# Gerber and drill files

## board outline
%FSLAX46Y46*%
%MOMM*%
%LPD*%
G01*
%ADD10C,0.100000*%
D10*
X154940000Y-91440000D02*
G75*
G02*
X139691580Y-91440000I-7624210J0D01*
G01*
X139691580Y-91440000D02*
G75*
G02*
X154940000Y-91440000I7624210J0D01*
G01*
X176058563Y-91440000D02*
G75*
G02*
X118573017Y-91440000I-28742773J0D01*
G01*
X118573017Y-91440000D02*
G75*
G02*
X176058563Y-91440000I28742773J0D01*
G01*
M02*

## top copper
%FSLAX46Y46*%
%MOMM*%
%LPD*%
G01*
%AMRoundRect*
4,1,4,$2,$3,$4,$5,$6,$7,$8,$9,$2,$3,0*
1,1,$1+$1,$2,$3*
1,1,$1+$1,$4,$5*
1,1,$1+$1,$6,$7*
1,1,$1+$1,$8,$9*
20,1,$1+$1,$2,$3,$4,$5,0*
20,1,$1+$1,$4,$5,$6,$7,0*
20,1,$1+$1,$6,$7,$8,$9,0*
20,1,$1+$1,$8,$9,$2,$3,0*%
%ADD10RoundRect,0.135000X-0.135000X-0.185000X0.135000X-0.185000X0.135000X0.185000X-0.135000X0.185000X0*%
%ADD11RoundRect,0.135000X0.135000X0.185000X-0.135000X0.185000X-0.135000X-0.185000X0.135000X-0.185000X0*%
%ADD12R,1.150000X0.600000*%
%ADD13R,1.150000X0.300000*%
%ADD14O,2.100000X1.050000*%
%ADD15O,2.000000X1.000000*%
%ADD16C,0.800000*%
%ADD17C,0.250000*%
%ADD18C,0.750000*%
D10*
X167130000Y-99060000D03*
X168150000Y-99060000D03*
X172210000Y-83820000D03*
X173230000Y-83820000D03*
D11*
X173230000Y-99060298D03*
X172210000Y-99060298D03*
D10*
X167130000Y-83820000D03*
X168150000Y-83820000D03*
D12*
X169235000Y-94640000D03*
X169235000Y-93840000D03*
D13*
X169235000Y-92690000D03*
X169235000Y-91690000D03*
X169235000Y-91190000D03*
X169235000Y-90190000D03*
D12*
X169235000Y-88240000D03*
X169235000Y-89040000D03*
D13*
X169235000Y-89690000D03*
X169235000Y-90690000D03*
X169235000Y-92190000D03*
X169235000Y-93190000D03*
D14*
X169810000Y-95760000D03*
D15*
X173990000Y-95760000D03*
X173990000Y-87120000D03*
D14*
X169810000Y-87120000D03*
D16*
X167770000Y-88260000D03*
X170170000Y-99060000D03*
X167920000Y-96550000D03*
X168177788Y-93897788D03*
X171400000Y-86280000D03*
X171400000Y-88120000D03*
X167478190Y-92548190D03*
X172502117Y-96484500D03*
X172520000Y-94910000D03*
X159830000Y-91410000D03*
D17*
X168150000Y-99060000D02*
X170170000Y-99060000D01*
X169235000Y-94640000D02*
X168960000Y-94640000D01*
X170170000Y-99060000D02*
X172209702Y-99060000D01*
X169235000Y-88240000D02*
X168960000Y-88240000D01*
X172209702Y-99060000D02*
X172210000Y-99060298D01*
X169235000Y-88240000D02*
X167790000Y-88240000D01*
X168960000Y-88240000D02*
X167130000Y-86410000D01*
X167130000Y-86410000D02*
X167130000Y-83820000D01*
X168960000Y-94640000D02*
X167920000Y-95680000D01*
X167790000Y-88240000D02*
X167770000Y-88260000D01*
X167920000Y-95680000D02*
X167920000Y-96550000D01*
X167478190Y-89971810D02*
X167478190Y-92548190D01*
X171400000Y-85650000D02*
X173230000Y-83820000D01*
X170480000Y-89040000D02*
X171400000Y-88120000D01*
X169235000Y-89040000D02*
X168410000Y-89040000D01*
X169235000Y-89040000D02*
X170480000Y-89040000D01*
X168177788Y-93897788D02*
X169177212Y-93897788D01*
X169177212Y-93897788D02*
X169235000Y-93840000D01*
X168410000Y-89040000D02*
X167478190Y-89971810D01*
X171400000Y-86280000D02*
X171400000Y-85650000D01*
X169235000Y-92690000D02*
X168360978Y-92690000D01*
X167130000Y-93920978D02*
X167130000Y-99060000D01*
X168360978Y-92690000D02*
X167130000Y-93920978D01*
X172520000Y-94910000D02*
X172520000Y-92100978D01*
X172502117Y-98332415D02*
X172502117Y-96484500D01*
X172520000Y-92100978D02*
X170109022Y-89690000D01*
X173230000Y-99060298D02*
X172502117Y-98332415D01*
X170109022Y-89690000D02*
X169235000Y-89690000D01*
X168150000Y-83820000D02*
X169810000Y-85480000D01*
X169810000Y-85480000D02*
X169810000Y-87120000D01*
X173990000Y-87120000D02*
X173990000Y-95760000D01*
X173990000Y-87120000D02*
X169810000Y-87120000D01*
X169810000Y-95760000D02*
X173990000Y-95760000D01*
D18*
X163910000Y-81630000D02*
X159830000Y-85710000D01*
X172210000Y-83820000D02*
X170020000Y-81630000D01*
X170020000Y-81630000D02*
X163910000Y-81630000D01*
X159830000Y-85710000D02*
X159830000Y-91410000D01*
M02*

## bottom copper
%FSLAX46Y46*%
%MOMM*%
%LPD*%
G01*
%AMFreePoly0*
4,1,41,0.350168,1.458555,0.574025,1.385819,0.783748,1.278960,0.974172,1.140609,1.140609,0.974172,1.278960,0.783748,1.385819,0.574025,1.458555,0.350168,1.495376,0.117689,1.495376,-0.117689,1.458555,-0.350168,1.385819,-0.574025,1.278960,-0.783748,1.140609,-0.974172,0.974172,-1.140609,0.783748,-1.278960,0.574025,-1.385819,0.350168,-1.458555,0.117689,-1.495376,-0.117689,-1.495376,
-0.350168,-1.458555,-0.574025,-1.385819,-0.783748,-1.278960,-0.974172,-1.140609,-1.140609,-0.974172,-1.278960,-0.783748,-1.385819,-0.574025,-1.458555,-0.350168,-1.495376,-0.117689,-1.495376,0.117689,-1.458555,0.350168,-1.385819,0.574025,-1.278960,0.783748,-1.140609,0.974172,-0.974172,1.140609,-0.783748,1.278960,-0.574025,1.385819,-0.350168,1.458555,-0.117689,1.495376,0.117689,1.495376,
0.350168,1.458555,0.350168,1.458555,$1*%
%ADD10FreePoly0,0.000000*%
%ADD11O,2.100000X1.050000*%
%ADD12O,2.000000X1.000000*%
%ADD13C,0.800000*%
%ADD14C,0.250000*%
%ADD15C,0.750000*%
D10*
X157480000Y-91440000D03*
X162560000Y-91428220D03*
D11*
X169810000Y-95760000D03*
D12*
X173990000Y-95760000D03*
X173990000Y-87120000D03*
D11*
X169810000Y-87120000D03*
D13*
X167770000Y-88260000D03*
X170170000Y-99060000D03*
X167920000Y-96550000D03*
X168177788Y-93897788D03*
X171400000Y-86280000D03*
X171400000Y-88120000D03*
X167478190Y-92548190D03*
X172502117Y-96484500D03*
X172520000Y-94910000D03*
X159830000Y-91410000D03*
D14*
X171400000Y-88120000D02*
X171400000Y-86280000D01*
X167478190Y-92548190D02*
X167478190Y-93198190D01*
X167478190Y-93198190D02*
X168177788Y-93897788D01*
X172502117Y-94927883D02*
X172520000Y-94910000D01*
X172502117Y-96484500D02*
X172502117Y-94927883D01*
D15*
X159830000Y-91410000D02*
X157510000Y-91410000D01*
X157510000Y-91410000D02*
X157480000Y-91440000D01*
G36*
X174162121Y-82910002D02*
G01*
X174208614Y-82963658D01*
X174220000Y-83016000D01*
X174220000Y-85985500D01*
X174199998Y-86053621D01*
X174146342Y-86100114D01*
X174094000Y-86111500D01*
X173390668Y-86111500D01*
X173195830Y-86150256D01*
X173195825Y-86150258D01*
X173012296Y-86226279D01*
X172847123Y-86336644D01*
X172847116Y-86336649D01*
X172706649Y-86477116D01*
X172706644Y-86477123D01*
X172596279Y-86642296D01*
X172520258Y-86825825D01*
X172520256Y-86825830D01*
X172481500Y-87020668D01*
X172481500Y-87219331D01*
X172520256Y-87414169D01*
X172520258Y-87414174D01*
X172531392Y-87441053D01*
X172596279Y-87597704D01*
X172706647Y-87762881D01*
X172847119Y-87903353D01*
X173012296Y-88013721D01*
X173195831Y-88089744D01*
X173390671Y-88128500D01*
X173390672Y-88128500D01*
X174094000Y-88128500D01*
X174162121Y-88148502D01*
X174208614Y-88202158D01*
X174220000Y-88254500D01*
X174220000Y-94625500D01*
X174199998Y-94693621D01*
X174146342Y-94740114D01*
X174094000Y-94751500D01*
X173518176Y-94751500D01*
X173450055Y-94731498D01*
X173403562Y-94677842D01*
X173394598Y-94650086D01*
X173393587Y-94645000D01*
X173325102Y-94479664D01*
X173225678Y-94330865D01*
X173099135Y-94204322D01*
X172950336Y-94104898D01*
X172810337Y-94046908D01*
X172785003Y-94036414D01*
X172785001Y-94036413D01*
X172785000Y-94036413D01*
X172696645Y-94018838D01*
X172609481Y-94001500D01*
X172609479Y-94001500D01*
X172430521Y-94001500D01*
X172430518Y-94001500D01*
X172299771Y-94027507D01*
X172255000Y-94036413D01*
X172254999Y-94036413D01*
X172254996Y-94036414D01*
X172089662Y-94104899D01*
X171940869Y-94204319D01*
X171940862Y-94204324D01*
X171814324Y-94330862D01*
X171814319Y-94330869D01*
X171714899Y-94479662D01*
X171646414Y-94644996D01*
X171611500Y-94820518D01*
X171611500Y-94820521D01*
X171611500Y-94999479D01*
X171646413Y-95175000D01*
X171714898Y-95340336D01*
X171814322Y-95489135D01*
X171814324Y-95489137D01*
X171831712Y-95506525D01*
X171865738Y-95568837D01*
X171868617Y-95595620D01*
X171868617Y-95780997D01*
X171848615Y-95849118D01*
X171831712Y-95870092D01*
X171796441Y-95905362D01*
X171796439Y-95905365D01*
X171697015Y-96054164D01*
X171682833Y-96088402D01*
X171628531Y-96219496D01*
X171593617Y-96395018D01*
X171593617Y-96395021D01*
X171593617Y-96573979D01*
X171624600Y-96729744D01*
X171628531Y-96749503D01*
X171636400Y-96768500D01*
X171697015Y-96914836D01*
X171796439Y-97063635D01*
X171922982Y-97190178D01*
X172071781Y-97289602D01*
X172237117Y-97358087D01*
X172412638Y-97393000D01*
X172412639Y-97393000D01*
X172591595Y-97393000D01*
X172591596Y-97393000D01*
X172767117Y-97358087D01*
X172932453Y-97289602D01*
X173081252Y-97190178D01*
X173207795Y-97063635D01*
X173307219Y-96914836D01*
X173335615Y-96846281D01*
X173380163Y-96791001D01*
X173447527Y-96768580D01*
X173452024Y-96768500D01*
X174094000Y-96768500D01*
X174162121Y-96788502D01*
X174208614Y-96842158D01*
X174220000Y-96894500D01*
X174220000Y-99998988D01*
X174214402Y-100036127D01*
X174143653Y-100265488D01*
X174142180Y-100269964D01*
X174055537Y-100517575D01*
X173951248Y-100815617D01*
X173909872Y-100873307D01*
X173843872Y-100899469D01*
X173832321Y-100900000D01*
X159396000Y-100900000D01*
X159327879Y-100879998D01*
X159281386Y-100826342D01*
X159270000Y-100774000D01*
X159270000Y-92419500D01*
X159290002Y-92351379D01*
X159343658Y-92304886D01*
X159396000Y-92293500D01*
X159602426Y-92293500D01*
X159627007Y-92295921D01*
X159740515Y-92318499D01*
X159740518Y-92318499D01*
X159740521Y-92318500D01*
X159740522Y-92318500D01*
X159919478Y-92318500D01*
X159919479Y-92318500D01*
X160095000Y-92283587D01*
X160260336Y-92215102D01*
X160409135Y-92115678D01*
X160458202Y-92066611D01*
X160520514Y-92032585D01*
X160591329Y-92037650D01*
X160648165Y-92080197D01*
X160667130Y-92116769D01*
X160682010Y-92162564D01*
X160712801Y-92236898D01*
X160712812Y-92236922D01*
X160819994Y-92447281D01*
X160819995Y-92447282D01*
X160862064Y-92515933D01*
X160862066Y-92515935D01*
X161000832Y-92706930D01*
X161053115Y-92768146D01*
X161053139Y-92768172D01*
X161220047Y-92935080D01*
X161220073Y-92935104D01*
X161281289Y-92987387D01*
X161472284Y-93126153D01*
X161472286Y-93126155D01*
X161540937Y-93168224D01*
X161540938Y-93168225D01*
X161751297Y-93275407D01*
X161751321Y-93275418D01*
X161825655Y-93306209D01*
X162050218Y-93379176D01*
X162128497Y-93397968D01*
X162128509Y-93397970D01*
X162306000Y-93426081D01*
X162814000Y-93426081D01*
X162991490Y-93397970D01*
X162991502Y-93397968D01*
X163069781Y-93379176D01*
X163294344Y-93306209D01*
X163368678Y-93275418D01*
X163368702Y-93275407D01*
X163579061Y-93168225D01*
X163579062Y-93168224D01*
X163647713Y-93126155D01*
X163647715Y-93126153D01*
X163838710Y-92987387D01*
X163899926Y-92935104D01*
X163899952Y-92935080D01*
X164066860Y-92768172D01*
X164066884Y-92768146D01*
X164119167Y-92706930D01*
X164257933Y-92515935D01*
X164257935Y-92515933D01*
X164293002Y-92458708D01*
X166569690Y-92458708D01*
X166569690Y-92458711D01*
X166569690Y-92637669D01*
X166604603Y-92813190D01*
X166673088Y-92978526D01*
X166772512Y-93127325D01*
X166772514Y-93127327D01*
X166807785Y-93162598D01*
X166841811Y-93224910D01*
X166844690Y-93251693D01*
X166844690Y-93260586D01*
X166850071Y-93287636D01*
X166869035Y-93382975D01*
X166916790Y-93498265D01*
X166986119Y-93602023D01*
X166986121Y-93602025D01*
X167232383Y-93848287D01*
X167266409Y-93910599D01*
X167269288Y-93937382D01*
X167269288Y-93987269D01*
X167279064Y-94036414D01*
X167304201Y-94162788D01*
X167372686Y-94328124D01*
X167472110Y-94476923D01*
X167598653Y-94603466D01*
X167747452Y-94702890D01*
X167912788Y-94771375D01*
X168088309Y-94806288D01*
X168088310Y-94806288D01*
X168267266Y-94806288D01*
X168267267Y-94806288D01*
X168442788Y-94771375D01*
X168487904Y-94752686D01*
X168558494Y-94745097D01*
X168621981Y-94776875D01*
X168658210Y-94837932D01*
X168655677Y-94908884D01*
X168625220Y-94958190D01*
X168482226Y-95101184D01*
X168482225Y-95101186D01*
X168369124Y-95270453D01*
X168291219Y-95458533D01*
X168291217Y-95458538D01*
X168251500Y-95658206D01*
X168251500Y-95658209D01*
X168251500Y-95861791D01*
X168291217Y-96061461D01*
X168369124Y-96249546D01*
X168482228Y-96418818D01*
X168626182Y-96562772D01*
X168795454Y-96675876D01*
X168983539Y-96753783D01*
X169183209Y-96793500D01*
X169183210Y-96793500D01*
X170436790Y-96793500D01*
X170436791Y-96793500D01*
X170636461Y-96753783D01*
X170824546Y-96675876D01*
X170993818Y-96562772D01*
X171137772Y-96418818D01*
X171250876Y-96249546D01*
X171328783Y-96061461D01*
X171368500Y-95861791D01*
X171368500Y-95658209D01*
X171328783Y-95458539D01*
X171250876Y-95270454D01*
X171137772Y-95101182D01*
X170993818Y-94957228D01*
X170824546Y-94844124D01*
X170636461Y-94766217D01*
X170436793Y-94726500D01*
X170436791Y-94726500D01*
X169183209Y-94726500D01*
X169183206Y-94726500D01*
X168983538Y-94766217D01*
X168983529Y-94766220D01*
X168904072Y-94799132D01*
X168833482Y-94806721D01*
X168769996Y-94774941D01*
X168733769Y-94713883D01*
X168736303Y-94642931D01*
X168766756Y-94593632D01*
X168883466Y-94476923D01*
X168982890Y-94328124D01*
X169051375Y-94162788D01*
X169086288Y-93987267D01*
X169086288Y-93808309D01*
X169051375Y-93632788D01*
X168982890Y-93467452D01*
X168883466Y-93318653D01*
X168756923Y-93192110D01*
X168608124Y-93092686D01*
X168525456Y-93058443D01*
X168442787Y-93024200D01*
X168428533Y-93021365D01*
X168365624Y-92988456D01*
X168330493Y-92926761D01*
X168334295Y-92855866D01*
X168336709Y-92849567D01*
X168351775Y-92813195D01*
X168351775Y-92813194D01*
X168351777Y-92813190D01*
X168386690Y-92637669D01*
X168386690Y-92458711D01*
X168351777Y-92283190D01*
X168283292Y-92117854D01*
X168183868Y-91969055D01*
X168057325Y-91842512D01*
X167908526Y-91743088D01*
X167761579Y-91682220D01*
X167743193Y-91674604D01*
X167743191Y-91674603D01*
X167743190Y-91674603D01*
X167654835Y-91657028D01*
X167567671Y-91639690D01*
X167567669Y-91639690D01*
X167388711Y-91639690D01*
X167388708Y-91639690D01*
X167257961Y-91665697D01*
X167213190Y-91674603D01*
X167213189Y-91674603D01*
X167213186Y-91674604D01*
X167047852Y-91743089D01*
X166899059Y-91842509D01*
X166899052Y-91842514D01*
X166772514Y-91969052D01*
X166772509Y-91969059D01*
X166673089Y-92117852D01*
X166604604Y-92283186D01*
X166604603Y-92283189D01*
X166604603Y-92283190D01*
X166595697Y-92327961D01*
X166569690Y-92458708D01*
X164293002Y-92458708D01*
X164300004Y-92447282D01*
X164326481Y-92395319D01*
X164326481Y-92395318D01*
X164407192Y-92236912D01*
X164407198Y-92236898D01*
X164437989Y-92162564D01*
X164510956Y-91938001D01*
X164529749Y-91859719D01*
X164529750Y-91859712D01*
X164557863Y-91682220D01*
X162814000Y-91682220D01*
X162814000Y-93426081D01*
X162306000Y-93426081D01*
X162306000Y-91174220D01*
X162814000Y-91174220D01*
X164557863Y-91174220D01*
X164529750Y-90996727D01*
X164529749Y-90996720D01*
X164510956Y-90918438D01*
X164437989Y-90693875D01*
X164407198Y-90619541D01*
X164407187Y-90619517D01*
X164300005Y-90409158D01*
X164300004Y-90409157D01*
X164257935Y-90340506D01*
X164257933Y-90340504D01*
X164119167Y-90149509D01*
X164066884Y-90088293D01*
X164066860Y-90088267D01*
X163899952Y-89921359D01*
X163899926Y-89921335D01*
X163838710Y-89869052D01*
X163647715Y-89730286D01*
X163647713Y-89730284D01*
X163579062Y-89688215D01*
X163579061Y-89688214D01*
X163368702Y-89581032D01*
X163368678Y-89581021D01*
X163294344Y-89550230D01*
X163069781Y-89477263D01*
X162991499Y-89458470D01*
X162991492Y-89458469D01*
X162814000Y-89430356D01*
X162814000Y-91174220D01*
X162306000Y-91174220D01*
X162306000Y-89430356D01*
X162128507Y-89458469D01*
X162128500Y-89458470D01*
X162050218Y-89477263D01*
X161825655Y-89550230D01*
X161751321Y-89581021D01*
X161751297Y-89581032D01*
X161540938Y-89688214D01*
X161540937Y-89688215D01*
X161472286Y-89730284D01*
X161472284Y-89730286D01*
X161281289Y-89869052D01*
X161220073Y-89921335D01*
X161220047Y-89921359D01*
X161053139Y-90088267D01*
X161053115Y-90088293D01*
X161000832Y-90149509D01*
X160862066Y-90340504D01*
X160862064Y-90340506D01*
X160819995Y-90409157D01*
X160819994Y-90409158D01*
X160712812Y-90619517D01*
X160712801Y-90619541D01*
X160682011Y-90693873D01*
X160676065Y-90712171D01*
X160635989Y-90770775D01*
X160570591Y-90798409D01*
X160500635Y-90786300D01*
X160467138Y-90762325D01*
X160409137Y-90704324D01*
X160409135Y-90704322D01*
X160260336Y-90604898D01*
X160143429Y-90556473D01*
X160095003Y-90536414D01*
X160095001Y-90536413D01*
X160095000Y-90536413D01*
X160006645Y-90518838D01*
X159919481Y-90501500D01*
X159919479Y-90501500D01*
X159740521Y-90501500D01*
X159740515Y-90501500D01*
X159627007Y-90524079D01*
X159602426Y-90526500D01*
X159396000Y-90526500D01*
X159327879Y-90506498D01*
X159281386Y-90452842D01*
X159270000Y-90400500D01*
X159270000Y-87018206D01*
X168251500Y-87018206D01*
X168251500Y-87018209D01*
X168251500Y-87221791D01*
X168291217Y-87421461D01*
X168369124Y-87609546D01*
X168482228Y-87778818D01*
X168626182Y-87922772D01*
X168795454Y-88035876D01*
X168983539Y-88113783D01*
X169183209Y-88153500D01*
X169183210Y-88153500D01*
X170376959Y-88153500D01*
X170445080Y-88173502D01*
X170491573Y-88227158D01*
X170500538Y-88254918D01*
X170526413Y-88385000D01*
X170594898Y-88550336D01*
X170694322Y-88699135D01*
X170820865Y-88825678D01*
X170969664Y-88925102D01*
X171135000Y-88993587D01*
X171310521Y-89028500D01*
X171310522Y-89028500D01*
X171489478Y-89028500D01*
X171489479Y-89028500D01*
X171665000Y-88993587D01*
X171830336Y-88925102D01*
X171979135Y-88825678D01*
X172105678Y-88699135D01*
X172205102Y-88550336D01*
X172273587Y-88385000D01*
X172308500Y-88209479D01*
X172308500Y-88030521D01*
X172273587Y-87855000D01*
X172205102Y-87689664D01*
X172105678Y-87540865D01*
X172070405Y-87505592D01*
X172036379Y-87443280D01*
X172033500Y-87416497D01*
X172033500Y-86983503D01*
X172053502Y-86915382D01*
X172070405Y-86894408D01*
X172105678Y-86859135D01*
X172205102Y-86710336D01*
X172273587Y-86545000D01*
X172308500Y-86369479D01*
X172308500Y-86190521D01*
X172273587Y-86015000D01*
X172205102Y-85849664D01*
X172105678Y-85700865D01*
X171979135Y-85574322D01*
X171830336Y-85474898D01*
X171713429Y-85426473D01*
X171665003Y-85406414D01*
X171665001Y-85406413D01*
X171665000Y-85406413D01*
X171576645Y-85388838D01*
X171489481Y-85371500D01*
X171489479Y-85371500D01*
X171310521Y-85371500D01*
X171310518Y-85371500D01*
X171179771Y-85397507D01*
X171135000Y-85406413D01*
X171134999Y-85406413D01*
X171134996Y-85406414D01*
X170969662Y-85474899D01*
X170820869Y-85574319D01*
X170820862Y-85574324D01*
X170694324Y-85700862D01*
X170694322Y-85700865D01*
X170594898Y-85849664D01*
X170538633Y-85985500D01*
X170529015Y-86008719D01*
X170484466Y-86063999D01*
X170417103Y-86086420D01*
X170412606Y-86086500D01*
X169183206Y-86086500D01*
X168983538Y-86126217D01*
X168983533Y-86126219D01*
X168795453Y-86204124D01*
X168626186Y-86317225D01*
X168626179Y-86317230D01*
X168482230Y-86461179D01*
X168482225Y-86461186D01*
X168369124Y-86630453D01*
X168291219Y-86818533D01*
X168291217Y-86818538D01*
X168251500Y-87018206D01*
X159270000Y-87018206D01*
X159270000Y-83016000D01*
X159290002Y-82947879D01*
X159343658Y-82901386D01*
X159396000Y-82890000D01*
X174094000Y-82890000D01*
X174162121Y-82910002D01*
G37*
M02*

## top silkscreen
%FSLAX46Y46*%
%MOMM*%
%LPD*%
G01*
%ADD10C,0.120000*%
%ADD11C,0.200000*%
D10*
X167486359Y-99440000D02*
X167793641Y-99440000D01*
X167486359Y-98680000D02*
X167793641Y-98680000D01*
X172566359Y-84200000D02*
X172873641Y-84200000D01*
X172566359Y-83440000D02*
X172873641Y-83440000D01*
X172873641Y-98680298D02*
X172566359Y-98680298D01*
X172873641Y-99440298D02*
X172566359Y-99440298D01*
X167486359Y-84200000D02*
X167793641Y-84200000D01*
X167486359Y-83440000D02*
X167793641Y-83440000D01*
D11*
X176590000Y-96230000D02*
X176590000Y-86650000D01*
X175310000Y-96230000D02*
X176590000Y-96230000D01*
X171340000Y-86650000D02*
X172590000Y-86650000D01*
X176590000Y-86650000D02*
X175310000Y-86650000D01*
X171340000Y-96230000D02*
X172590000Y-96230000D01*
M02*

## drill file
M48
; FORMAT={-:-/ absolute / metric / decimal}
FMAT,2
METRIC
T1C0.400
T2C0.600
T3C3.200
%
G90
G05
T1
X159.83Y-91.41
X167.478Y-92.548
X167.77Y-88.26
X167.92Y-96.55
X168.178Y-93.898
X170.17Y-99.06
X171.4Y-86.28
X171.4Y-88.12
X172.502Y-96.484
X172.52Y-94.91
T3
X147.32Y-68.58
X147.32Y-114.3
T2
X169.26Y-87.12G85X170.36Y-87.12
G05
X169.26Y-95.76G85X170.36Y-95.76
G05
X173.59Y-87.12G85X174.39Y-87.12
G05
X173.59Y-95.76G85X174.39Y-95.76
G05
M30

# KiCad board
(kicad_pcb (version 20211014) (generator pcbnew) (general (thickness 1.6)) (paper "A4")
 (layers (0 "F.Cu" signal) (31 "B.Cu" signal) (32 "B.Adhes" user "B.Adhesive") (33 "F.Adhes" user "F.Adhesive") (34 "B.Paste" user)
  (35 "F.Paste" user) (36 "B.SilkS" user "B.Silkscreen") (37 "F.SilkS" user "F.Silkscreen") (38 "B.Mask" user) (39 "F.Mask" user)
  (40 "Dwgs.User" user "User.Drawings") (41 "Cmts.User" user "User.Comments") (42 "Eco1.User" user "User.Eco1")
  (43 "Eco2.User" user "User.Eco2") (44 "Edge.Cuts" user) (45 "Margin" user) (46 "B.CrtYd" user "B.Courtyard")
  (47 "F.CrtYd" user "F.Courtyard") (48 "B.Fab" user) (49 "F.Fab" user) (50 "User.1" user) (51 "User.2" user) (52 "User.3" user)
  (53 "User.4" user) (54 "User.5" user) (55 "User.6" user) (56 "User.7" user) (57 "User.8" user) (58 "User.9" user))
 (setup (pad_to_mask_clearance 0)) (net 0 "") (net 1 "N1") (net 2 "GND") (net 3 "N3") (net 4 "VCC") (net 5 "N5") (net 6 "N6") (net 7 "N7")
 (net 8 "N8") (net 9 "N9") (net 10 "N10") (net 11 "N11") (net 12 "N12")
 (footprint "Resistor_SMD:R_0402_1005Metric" (layer "F.Cu") (at 167.64 99.06)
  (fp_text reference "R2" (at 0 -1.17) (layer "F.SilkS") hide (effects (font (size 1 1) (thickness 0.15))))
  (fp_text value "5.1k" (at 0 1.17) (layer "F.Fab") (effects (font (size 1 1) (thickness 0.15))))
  (fp_line (start -0.153641 0.38) (end 0.153641 0.38) (layer "F.SilkS") (width 0.12))
  (fp_line (start -0.153641 -0.38) (end 0.153641 -0.38) (layer "F.SilkS") (width 0.12))
  (pad "1" smd roundrect (at -0.51 0) (size 0.54 0.64) (layers "F.Cu" "F.Paste" "F.Mask") (roundrect_rratio 0.25) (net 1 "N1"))
  (pad "2" smd roundrect (at 0.51 0) (size 0.54 0.64) (layers "F.Cu" "F.Paste" "F.Mask") (roundrect_rratio 0.25) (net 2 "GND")))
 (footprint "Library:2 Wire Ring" (layer "F.Cu") (at 147.32 91.44)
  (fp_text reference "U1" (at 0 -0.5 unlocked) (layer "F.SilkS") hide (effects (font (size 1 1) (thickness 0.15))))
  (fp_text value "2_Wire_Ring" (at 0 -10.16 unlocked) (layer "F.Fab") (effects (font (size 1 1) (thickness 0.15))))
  (pad "1" smd custom (at 10.16 0) (size 3 3) (layers "B.Cu" "B.Mask") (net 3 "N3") (options (clearance outline) (anchor circle))
   (primitives))
  (pad "2" smd custom (at 15.24 -0.01178) (size 3 3) (layers "B.Cu" "B.Mask") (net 2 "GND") (options (clearance outline) (anchor circle))
   (primitives)))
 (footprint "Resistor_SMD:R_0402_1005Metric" (layer "F.Cu") (at 172.72 83.82)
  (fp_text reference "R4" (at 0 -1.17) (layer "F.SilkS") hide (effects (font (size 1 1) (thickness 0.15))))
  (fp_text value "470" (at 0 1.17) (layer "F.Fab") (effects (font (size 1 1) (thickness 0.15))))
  (fp_line (start -0.153641 0.38) (end 0.153641 0.38) (layer "F.SilkS") (width 0.12))
  (fp_line (start -0.153641 -0.38) (end 0.153641 -0.38) (layer "F.SilkS") (width 0.12))
  (pad "1" smd roundrect (at -0.51 0) (size 0.54 0.64) (layers "F.Cu" "F.Paste" "F.Mask") (roundrect_rratio 0.25) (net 3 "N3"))
  (pad "2" smd roundrect (at 0.51 0) (size 0.54 0.64) (layers "F.Cu" "F.Paste" "F.Mask") (roundrect_rratio 0.25) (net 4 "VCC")))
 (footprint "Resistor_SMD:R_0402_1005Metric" (layer "F.Cu") (at 172.72 99.060298 180)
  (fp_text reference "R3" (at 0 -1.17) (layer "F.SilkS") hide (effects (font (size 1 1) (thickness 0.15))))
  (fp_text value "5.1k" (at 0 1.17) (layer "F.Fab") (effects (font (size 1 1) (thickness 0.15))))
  (fp_line (start -0.153641 0.38) (end 0.153641 0.38) (layer "F.SilkS") (width 0.12))
  (fp_line (start -0.153641 -0.38) (end 0.153641 -0.38) (layer "F.SilkS") (width 0.12))
  (pad "1" smd roundrect (at -0.51 0 180) (size 0.54 0.64) (layers "F.Cu" "F.Paste" "F.Mask") (roundrect_rratio 0.25) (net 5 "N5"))
  (pad "2" smd roundrect (at 0.51 0 180) (size 0.54 0.64) (layers "F.Cu" "F.Paste" "F.Mask") (roundrect_rratio 0.25) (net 2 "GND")))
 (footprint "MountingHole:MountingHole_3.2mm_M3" (layer "F.Cu") (at 147.32 68.58)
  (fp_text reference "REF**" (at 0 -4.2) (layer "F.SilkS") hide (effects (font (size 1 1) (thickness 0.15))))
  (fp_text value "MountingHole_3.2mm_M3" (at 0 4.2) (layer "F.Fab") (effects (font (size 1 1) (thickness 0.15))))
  (pad "" np_thru_hole circle (at 0 0) (size 3.2 3.2) (drill 3.2) (layers *.Cu *.Mask)))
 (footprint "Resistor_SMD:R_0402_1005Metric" (layer "F.Cu") (at 167.64 83.82)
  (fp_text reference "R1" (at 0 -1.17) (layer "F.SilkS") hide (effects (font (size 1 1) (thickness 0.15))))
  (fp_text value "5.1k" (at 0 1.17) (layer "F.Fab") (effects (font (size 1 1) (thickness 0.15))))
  (fp_line (start -0.153641 0.38) (end 0.153641 0.38) (layer "F.SilkS") (width 0.12))
  (fp_line (start -0.153641 -0.38) (end 0.153641 -0.38) (layer "F.SilkS") (width 0.12))
  (pad "1" smd roundrect (at -0.51 0) (size 0.54 0.64) (layers "F.Cu" "F.Paste" "F.Mask") (roundrect_rratio 0.25) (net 2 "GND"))
  (pad "2" smd roundrect (at 0.51 0) (size 0.54 0.64) (layers "F.Cu" "F.Paste" "F.Mask") (roundrect_rratio 0.25) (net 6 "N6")))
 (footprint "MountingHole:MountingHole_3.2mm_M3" (layer "F.Cu") (at 147.32 114.3)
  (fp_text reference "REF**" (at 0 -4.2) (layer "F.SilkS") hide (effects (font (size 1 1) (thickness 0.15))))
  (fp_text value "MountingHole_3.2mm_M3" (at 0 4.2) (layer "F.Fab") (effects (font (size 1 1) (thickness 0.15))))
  (pad "" np_thru_hole circle (at 0 0) (size 3.2 3.2) (drill 3.2) (layers *.Cu *.Mask)))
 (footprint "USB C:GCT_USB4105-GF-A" (layer "F.Cu") (at 173.99 91.44 90)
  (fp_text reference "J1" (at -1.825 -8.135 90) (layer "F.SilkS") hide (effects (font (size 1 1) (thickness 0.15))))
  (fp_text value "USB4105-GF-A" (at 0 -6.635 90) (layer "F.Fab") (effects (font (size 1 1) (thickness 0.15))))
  (fp_line (start -4.79 2.6) (end 4.79 2.6) (layer "F.SilkS") (width 0.2))
  (fp_line (start -4.79 1.32) (end -4.79 2.6) (layer "F.SilkS") (width 0.2))
  (fp_line (start 4.79 -2.65) (end 4.79 -1.4) (layer "F.SilkS") (width 0.2))
  (fp_line (start 4.79 2.6) (end 4.79 1.32) (layer "F.SilkS") (width 0.2))
  (fp_line (start -4.79 -2.65) (end -4.79 -1.4) (layer "F.SilkS") (width 0.2))
  (pad "A1_B12" smd rect (at -3.2 -4.755 90) (size 0.6 1.15) (layers "F.Cu" "F.Paste" "F.Mask") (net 2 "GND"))
  (pad "A4_B9" smd rect (at -2.4 -4.755 90) (size 0.6 1.15) (layers "F.Cu" "F.Paste" "F.Mask") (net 4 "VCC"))
  (pad "A5" smd rect (at -1.25 -4.755 90) (size 0.3 1.15) (layers "F.Cu" "F.Paste" "F.Mask") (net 1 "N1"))
  (pad "A6" smd rect (at -0.25 -4.755 90) (size 0.3 1.15) (layers "F.Cu" "F.Paste" "F.Mask") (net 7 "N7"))
  (pad "A7" smd rect (at 0.25 -4.755 90) (size 0.3 1.15) (layers "F.Cu" "F.Paste" "F.Mask") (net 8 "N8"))
  (pad "A8" smd rect (at 1.25 -4.755 90) (size 0.3 1.15) (layers "F.Cu" "F.Paste" "F.Mask") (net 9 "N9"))
  (pad "B1_A12" smd rect (at 3.2 -4.755 90) (size 0.6 1.15) (layers "F.Cu" "F.Paste" "F.Mask") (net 2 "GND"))
  (pad "B4_A9" smd rect (at 2.4 -4.755 90) (size 0.6 1.15) (layers "F.Cu" "F.Paste" "F.Mask") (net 4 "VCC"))
  (pad "B5" smd rect (at 1.75 -4.755 90) (size 0.3 1.15) (layers "F.Cu" "F.Paste" "F.Mask") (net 5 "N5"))
  (pad "B6" smd rect (at 0.75 -4.755 90) (size 0.3 1.15) (layers "F.Cu" "F.Paste" "F.Mask") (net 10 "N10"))
  (pad "B7" smd rect (at -0.75 -4.755 90) (size 0.3 1.15) (layers "F.Cu" "F.Paste" "F.Mask") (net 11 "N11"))
  (pad "B8" smd rect (at -1.75 -4.755 90) (size 0.3 1.15) (layers "F.Cu" "F.Paste" "F.Mask") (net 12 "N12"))
  (pad "S1" thru_hole oval (at -4.32 -4.18 90) (size 1.05 2.1) (drill oval 0.6 1.7) (layers *.Cu *.Mask) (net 6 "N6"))
  (pad "S2" thru_hole oval (at -4.32 0 90) (size 1 2) (drill oval 0.6 1.4) (layers *.Cu *.Mask) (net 6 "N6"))
  (pad "S3" thru_hole oval (at 4.32 0 90) (size 1 2) (drill oval 0.6 1.4) (layers *.Cu *.Mask) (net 6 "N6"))
  (pad "S4" thru_hole oval (at 4.32 -4.18 90) (size 1.05 2.1) (drill oval 0.6 1.7) (layers *.Cu *.Mask) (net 6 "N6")))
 (gr_circle (center 147.31579 91.44) (end 154.94 91.44) (layer "Edge.Cuts") (width 0.1) (fill none))
 (gr_circle (center 147.31579 91.44) (end 167.64 71.11579) (layer "Edge.Cuts") (width 0.1) (fill none))
 (segment (start 168.15 99.06) (end 170.17 99.06) (width 0.25) (layer "F.Cu") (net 2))
 (segment (start 169.235 94.64) (end 168.96 94.64) (width 0.25) (layer "F.Cu") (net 2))
 (segment (start 170.17 99.06) (end 172.209702 99.06) (width 0.25) (layer "F.Cu") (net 2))
 (segment (start 169.235 88.24) (end 168.96 88.24) (width 0.25) (layer "F.Cu") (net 2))
 (segment (start 172.209702 99.06) (end 172.21 99.060298) (width 0.25) (layer "F.Cu") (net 2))
 (segment (start 169.235 88.24) (end 167.79 88.24) (width 0.25) (layer "F.Cu") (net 2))
 (segment (start 168.96 88.24) (end 167.13 86.41) (width 0.25) (layer "F.Cu") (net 2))
 (segment (start 167.13 86.41) (end 167.13 83.82) (width 0.25) (layer "F.Cu") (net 2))
 (segment (start 168.96 94.64) (end 167.92 95.68) (width 0.25) (layer "F.Cu") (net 2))
 (segment (start 167.79 88.24) (end 167.77 88.26) (width 0.25) (layer "F.Cu") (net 2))
 (segment (start 167.92 95.68) (end 167.92 96.55) (width 0.25) (layer "F.Cu") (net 2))
 (via (at 167.77 88.26) (size 0.8) (drill 0.4) (layers "F.Cu" "B.Cu") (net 2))
 (via (at 170.17 99.06) (size 0.8) (drill 0.4) (layers "F.Cu" "B.Cu") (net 2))
 (via (at 167.92 96.55) (size 0.8) (drill 0.4) (layers "F.Cu" "B.Cu") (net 2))
 (segment (start 167.47819 89.97181) (end 167.47819 92.54819) (width 0.25) (layer "F.Cu") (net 4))
 (segment (start 171.4 85.65) (end 173.23 83.82) (width 0.25) (layer "F.Cu") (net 4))
 (segment (start 170.48 89.04) (end 171.4 88.12) (width 0.25) (layer "F.Cu") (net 4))
 (segment (start 169.235 89.04) (end 168.41 89.04) (width 0.25) (layer "F.Cu") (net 4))
 (segment (start 169.235 89.04) (end 170.48 89.04) (width 0.25) (layer "F.Cu") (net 4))
 (segment (start 168.177788 93.897788) (end 169.177212 93.897788) (width 0.25) (layer "F.Cu") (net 4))
 (segment (start 169.177212 93.897788) (end 169.235 93.84) (width 0.25) (layer "F.Cu") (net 4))
 (segment (start 168.41 89.04) (end 167.47819 89.97181) (width 0.25) (layer "F.Cu") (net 4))
 (segment (start 171.4 86.28) (end 171.4 85.65) (width 0.25) (layer "F.Cu") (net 4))
 (via (at 168.177788 93.897788) (size 0.8) (drill 0.4) (layers "F.Cu" "B.Cu") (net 4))
 (via (at 171.4 86.28) (size 0.8) (drill 0.4) (layers "F.Cu" "B.Cu") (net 4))
 (via (at 171.4 88.12) (size 0.8) (drill 0.4) (layers "F.Cu" "B.Cu") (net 4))
 (via (at 167.47819 92.54819) (size 0.8) (drill 0.4) (layers "F.Cu" "B.Cu") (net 4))
 (segment (start 171.4 88.12) (end 171.4 86.28) (width 0.25) (layer "B.Cu") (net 4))
 (segment (start 167.47819 92.54819) (end 167.47819 93.19819) (width 0.25) (layer "B.Cu") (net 4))
 (segment (start 167.47819 93.19819) (end 168.177788 93.897788) (width 0.25) (layer "B.Cu") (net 4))
 (segment (start 169.235 92.69) (end 168.360978 92.69) (width 0.25) (layer "F.Cu") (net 1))
 (segment (start 167.13 93.920978) (end 167.13 99.06) (width 0.25) (layer "F.Cu") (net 1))
 (segment (start 168.360978 92.69) (end 167.13 93.920978) (width 0.25) (layer "F.Cu") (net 1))
 (segment (start 172.52 94.91) (end 172.52 92.100978) (width 0.25) (layer "F.Cu") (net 5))
 (segment (start 172.502117 98.332415) (end 172.502117 96.4845) (width 0.25) (layer "F.Cu") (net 5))
 (segment (start 172.52 92.100978) (end 170.109022 89.69) (width 0.25) (layer "F.Cu") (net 5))
 (segment (start 173.23 99.060298) (end 172.502117 98.332415) (width 0.25) (layer "F.Cu") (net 5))
 (segment (start 170.109022 89.69) (end 169.235 89.69) (width 0.25) (layer "F.Cu") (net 5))
 (via (at 172.502117 96.4845) (size 0.8) (drill 0.4) (layers "F.Cu" "B.Cu") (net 5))
 (via (at 172.52 94.91) (size 0.8) (drill 0.4) (layers "F.Cu" "B.Cu") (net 5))
 (segment (start 172.502117 94.927883) (end 172.52 94.91) (width 0.25) (layer "B.Cu") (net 5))
 (segment (start 172.502117 96.4845) (end 172.502117 94.927883) (width 0.25) (layer "B.Cu") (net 5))
 (segment (start 168.15 83.82) (end 169.81 85.48) (width 0.25) (layer "F.Cu") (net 6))
 (segment (start 169.81 85.48) (end 169.81 87.12) (width 0.25) (layer "F.Cu") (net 6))
 (segment (start 173.99 87.12) (end 173.99 95.76) (width 0.25) (layer "F.Cu") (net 6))
 (segment (start 173.99 87.12) (end 169.81 87.12) (width 0.25) (layer "F.Cu") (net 6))
 (segment (start 169.81 95.76) (end 173.99 95.76) (width 0.25) (layer "F.Cu") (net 6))
 (segment (start 163.91 81.63) (end 159.83 85.71) (width 0.75) (layer "F.Cu") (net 3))
 (segment (start 172.21 83.82) (end 170.02 81.63) (width 0.75) (layer "F.Cu") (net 3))
 (segment (start 170.02 81.63) (end 163.91 81.63) (width 0.75) (layer "F.Cu") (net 3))
 (segment (start 159.83 85.71) (end 159.83 91.41) (width 0.75) (layer "F.Cu") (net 3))
 (via (at 159.83 91.41) (size 0.8) (drill 0.4) (layers "F.Cu" "B.Cu") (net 3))
 (segment (start 159.83 91.41) (end 157.51 91.41) (width 0.75) (layer "B.Cu") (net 3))
 (segment (start 157.51 91.41) (end 157.48 91.44) (width 0.75) (layer "B.Cu") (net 3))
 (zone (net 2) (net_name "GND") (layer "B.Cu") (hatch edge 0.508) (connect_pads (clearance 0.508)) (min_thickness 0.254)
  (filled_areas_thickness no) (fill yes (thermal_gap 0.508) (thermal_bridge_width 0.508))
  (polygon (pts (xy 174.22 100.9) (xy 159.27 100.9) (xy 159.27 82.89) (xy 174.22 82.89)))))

